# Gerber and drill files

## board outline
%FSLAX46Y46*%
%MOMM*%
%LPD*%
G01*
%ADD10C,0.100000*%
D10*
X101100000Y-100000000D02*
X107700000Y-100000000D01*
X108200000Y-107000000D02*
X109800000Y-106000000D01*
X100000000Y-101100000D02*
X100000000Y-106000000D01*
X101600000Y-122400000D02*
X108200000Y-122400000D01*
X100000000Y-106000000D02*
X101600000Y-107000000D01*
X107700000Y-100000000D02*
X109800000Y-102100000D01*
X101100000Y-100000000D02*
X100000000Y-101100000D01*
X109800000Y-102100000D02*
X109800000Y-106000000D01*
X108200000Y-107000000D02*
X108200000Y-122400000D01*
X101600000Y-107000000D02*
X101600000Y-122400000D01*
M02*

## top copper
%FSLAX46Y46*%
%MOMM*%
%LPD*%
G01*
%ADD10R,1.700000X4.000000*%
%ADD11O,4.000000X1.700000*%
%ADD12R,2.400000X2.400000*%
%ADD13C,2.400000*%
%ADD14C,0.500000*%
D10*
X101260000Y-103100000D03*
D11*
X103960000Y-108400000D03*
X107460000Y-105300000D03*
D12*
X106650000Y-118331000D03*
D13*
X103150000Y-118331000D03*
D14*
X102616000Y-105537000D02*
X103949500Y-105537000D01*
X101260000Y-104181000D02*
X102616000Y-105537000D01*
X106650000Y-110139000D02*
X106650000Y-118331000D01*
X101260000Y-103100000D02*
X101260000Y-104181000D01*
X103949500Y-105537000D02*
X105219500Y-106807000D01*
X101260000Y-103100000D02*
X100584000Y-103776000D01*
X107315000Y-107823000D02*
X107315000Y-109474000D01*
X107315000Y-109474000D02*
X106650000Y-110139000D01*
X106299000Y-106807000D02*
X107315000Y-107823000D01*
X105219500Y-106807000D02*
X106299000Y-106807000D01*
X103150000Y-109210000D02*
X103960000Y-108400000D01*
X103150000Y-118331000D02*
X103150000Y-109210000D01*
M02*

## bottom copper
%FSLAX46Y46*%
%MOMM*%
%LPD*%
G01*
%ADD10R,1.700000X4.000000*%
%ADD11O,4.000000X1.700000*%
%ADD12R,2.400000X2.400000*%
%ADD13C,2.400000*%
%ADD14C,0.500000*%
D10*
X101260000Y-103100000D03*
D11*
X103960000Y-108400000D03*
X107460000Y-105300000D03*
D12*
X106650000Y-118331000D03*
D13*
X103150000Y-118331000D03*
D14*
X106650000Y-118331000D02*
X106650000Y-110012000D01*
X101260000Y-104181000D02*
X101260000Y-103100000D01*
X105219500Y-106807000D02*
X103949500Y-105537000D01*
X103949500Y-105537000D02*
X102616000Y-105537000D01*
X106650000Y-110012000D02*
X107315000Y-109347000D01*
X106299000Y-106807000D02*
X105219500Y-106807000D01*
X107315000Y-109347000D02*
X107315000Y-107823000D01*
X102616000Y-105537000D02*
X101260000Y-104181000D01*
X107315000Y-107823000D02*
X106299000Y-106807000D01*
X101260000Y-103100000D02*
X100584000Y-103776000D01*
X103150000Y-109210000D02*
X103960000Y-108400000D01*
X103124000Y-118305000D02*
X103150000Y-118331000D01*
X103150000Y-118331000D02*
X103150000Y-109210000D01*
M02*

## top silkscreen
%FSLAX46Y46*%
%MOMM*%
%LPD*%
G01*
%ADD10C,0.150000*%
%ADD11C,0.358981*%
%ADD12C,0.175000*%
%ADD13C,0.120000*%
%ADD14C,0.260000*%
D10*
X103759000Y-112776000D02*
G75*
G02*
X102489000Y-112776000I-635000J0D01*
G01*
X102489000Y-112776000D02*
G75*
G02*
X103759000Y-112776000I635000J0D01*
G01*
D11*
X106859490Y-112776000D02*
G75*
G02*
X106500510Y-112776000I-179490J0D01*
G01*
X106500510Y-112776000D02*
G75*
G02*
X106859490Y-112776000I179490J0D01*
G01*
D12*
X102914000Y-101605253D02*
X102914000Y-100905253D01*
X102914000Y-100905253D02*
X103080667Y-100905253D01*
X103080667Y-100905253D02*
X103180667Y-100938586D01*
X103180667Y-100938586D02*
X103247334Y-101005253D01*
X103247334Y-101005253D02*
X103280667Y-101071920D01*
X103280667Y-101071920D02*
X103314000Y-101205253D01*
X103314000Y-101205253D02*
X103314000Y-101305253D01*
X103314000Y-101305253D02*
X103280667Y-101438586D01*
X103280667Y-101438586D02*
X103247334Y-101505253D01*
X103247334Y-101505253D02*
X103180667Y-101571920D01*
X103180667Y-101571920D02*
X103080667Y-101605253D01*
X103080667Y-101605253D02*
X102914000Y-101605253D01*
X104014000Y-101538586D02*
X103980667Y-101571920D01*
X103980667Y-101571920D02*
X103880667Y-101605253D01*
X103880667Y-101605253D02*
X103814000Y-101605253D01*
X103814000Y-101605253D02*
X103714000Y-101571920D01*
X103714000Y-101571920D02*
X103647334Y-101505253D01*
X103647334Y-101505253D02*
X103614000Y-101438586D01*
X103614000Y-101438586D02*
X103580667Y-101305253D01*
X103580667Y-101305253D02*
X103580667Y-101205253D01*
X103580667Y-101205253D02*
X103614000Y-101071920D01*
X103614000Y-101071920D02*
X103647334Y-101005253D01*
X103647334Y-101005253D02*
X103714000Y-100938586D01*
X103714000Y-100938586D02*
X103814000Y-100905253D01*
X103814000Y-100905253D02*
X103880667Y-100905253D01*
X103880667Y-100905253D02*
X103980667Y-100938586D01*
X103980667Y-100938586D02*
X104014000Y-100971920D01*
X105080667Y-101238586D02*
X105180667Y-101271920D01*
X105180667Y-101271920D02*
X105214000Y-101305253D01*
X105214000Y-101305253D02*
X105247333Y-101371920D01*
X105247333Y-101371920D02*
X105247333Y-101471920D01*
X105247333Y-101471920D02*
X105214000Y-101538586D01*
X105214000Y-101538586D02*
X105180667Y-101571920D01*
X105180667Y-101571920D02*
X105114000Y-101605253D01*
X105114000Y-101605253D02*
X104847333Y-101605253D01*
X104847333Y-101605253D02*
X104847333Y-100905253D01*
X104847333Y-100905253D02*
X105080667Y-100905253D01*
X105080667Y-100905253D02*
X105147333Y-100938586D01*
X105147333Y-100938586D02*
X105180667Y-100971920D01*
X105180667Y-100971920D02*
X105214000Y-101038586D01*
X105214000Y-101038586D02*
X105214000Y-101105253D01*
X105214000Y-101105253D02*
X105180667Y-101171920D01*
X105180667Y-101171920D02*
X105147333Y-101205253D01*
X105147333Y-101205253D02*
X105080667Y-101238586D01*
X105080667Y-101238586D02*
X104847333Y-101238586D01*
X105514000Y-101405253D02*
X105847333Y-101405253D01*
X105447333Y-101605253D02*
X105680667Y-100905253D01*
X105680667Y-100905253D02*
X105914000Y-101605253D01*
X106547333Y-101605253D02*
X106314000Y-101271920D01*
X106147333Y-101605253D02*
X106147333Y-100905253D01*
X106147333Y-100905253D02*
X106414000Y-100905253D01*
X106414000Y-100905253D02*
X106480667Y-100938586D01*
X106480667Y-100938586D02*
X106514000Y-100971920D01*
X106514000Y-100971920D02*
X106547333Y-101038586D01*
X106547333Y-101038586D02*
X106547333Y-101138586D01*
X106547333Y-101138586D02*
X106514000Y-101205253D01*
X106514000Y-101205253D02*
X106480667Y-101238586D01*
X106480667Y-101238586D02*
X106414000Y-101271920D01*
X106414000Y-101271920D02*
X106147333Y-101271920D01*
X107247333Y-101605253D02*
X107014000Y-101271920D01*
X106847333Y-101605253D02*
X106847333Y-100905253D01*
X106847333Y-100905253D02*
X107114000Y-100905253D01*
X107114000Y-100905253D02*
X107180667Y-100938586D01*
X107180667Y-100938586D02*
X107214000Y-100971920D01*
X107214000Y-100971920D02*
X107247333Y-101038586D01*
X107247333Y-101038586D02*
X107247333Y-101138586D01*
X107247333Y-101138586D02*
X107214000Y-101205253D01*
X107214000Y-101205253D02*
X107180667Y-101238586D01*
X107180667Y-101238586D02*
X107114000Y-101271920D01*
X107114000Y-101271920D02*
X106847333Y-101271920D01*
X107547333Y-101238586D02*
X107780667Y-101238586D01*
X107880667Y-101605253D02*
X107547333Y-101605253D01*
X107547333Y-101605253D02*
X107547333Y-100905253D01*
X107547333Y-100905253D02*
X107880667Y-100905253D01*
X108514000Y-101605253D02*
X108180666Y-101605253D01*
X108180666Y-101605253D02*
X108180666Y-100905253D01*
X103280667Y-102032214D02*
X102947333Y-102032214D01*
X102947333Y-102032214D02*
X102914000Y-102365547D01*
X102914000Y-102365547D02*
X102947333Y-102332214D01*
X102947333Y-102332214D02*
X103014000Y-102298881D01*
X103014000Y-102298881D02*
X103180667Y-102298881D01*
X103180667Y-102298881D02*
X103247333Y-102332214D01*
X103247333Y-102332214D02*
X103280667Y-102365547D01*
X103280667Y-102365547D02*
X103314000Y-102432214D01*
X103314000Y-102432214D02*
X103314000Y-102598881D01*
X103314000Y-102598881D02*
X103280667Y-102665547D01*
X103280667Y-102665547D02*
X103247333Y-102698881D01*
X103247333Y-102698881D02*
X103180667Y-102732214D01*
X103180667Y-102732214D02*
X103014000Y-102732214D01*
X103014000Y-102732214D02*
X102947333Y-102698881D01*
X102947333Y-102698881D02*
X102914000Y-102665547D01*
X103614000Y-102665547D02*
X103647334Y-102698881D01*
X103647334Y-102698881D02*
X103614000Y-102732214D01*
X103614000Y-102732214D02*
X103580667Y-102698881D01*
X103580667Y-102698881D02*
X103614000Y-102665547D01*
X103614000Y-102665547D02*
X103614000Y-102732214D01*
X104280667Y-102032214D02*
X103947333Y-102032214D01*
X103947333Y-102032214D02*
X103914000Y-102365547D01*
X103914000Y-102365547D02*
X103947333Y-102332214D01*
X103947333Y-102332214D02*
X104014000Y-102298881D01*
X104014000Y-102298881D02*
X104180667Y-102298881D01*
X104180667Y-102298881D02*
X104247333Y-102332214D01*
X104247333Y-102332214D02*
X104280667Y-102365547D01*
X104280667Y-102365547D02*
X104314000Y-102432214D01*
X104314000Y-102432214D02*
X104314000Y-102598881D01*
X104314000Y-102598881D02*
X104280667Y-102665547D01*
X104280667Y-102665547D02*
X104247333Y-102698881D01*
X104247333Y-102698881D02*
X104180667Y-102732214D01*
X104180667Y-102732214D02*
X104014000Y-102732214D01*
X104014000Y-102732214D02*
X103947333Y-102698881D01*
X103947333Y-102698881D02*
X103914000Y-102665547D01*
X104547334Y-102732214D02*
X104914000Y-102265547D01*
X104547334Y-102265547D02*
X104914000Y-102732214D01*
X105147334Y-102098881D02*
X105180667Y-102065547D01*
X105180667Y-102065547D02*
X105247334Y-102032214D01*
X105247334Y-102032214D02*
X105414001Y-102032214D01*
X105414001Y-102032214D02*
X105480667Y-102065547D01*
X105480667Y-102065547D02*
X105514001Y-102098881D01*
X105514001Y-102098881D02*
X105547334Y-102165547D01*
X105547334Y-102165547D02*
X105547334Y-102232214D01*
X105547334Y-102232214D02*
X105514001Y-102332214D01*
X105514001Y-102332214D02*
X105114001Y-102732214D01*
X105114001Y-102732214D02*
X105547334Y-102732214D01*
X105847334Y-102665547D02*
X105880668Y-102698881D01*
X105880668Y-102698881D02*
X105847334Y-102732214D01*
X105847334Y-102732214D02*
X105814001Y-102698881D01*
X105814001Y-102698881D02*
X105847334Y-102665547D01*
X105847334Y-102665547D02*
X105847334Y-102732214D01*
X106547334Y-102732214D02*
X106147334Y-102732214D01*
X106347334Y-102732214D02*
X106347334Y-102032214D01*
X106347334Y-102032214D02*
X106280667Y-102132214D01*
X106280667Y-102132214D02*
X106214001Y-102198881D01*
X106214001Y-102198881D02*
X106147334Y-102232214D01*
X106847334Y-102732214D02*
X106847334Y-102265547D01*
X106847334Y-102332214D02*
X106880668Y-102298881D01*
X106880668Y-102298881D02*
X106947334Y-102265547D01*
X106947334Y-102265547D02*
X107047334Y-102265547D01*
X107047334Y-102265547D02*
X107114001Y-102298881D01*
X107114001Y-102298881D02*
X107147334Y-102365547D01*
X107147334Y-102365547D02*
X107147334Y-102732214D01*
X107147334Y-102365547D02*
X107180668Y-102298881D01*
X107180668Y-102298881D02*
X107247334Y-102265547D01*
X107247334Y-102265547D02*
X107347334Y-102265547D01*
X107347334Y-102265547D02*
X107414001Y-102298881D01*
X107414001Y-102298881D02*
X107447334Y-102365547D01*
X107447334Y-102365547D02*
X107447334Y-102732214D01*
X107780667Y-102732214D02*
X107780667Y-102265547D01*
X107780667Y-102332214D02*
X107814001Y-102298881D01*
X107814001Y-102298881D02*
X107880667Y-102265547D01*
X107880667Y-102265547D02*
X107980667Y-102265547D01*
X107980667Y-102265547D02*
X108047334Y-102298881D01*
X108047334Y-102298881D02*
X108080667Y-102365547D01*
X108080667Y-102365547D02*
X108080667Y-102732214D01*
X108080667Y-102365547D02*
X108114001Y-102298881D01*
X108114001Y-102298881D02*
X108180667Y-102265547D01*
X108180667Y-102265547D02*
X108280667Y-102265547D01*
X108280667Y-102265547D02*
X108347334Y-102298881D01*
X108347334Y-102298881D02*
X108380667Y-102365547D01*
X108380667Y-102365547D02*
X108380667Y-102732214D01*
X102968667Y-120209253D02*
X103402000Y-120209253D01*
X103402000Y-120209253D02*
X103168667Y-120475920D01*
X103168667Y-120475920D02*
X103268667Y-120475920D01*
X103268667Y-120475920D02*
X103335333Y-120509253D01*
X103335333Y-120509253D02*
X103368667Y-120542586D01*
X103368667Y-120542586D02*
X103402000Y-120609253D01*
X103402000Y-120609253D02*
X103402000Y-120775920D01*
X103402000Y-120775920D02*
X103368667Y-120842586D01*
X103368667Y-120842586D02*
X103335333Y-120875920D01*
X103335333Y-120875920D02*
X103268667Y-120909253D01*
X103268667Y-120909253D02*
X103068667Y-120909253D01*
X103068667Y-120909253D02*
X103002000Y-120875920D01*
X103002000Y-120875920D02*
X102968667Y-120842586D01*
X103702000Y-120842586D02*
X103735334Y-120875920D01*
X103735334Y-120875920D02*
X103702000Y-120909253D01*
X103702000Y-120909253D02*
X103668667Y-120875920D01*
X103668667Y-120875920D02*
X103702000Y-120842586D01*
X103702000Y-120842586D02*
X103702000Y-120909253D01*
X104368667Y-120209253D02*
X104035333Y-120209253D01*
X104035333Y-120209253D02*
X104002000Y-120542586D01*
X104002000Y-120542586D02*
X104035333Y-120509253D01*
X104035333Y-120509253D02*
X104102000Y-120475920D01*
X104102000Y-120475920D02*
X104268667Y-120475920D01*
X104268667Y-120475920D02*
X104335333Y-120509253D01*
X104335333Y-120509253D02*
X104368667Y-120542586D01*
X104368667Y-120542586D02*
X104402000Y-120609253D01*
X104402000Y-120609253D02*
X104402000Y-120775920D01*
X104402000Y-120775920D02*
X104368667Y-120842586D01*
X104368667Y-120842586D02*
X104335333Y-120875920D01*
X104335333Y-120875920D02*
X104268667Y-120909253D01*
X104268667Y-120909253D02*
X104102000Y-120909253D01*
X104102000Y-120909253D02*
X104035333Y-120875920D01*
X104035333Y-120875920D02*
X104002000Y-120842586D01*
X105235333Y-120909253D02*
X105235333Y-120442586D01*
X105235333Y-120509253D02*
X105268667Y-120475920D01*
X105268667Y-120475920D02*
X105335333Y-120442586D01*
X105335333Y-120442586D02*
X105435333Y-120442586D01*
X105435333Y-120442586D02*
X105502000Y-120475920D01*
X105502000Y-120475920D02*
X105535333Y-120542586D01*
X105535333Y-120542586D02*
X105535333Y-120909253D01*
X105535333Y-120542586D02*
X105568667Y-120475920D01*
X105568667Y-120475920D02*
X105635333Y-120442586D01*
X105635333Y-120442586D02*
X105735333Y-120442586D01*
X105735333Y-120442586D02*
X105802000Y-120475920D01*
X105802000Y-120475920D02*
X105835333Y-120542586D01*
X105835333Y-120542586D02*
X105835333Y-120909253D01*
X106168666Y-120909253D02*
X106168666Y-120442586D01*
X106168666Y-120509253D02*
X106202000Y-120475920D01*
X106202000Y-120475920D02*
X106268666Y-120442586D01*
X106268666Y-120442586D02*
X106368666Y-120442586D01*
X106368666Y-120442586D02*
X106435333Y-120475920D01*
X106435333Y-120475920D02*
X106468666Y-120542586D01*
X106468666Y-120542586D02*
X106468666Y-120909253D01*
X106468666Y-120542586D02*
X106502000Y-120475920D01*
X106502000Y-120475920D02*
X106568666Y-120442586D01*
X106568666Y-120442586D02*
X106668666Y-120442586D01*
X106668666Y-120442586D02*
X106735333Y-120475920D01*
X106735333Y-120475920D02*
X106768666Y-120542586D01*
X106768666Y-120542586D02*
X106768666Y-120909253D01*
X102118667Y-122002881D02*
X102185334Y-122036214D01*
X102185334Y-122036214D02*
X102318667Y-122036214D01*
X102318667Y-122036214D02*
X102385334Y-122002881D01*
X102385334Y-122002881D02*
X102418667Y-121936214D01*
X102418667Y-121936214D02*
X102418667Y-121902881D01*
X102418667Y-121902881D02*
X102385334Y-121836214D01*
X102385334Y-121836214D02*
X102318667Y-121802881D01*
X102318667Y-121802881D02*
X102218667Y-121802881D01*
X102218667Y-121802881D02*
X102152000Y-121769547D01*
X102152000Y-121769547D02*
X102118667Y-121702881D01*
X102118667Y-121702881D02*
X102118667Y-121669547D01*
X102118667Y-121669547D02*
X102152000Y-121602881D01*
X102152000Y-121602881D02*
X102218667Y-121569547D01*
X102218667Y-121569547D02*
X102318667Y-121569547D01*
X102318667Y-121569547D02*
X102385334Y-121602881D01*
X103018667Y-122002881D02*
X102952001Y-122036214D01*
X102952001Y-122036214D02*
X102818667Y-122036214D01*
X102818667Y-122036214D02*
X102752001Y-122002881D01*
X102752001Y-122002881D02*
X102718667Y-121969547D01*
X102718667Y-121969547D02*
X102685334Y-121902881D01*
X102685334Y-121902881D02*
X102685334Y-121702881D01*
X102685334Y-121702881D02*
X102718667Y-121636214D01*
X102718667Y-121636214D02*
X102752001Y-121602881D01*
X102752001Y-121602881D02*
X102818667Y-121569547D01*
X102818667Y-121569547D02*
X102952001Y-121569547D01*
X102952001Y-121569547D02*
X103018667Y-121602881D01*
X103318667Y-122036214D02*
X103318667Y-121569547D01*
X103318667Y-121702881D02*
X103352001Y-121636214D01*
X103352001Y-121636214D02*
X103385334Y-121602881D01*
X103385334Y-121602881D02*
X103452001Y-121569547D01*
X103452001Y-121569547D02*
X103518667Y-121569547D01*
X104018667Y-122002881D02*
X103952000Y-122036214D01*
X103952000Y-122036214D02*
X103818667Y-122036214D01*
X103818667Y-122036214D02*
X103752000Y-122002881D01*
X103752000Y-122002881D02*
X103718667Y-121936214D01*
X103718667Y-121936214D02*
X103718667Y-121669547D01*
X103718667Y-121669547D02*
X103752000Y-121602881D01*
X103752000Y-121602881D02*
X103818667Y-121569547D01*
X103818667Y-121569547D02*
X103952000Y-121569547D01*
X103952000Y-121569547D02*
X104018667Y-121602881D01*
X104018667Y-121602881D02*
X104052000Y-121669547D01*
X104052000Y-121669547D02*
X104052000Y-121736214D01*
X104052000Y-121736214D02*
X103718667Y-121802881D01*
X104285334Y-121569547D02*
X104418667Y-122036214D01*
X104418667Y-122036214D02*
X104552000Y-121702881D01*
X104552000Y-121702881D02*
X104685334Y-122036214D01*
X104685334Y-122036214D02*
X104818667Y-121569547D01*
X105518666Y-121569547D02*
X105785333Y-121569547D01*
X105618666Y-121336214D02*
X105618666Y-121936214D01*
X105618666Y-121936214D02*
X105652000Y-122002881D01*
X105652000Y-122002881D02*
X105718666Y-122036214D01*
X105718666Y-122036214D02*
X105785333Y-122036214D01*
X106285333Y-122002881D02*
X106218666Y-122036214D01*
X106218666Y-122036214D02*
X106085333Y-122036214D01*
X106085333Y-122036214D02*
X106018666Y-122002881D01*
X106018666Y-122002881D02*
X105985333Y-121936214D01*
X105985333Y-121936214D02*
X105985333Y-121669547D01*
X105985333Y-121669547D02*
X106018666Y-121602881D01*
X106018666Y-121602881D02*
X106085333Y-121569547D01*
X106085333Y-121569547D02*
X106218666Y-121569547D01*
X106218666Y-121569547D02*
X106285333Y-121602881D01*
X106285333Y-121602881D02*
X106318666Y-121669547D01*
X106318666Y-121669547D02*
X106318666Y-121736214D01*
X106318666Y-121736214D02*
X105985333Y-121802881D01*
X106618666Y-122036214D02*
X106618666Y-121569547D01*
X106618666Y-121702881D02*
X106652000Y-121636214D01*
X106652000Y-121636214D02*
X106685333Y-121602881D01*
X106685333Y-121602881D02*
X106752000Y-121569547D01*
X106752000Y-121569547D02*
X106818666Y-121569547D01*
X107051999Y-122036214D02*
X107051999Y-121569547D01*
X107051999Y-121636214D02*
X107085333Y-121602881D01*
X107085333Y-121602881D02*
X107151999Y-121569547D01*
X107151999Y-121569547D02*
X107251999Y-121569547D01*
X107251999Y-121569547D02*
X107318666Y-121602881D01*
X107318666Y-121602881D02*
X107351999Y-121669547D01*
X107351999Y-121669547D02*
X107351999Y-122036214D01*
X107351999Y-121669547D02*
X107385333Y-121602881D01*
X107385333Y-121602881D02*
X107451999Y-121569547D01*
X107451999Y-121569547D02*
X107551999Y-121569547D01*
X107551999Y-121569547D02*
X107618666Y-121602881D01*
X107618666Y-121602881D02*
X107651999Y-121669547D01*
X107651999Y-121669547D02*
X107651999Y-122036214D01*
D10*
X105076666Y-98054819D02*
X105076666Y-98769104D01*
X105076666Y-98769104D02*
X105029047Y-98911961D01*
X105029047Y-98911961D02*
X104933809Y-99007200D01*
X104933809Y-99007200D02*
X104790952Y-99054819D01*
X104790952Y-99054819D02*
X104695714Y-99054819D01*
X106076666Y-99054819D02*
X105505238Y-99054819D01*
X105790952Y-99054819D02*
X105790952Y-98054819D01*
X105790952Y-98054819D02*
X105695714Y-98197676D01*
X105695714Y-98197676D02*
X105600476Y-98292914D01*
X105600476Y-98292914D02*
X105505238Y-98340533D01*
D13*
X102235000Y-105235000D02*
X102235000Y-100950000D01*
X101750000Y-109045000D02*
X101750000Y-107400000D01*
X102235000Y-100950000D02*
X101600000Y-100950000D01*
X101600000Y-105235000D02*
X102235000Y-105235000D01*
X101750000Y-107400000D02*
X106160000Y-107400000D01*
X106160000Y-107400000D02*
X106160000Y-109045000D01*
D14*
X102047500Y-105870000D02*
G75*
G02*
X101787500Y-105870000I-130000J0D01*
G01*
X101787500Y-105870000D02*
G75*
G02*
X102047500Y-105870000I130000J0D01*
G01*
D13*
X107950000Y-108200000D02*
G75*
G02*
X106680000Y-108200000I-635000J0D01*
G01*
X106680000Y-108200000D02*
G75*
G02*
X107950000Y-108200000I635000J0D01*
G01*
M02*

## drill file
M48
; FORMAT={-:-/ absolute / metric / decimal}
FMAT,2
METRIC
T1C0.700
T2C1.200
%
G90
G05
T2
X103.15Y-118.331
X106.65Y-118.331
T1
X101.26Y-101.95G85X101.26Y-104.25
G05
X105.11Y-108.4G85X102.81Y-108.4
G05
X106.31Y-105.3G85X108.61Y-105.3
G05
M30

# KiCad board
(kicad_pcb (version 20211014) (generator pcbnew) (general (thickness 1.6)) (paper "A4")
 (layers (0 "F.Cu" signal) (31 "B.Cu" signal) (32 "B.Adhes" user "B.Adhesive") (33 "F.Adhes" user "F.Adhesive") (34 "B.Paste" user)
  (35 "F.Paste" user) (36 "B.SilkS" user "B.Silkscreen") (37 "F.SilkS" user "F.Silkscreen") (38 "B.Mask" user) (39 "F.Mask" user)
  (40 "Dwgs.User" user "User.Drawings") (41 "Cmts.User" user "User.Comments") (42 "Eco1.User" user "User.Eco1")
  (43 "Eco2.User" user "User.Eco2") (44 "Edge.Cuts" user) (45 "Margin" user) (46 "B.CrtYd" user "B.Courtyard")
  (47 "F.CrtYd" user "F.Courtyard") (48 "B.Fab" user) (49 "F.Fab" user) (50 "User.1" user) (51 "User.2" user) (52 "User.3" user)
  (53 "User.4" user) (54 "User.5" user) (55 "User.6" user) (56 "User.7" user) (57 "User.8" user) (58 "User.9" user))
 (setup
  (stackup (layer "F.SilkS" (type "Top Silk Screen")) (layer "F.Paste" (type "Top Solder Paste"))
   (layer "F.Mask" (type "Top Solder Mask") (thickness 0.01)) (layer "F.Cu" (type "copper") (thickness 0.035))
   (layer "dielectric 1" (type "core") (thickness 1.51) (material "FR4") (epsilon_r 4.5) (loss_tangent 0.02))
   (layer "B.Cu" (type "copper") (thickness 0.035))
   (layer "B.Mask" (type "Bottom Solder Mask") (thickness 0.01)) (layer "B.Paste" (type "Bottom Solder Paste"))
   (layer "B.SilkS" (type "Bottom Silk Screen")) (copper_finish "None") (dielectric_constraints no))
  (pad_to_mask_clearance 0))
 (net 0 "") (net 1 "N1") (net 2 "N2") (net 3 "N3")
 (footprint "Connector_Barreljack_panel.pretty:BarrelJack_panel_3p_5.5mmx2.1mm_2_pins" (layer "F.Cu") (at 105.41 104.6)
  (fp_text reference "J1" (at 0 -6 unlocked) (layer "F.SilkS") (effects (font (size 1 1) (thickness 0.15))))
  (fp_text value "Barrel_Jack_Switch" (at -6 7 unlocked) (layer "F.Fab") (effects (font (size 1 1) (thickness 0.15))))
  (fp_line (start -3.175 0.635) (end -3.175 -3.65) (layer "F.SilkS") (width 0.12))
  (fp_line (start -3.66 4.445) (end -3.66 2.8) (layer "F.SilkS") (width 0.12))
  (fp_line (start -3.175 -3.65) (end -3.81 -3.65) (layer "F.SilkS") (width 0.12))
  (fp_line (start -3.81 0.635) (end -3.175 0.635) (layer "F.SilkS") (width 0.12))
  (fp_line (start -3.66 2.8) (end 0.75 2.8) (layer "F.SilkS") (width 0.12))
  (fp_line (start 0.75 2.8) (end 0.75 4.445) (layer "F.SilkS") (width 0.12))
  (fp_circle (center -3.4925 1.27) (end -3.2925 1.27) (layer "F.SilkS") (width 0.12) (fill solid))
  (fp_circle (center 1.905 3.6) (end 2.54 3.6) (layer "F.SilkS") (width 0.12) (fill none))
  (pad "1" thru_hole rect (at -4.15 -1.5) (size 1.7 4) (drill oval 0.7 3) (layers *.Cu *.Mask) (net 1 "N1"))
  (pad "2" thru_hole oval (at -1.45 3.8 270) (size 1.7 4) (drill oval 0.7 3) (layers *.Cu *.Mask) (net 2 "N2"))
  (pad "3" thru_hole oval (at 2.05 0.7 90) (size 1.7 4) (drill oval 0.7 3) (layers *.Cu *.Mask) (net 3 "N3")))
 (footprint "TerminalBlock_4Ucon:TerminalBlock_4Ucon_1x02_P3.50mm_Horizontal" (layer "B.Cu") (at 106.65 118.331 180)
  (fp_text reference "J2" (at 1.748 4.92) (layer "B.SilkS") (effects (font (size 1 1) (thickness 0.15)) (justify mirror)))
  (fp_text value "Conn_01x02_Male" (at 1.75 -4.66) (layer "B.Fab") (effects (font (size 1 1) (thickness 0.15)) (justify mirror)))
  (pad "1" thru_hole rect (at 0 0 180) (size 2.4 2.4) (drill 1.2) (layers *.Cu *.Mask) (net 1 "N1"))
  (pad "2" thru_hole circle (at 3.5 0 180) (size 2.4 2.4) (drill 1.2) (layers *.Cu *.Mask) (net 2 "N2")))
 (gr_circle (center 103.124 112.776) (end 103.632 112.395) (layer "F.SilkS") (width 0.15) (fill none))
 (gr_circle (center 106.68 112.776) (end 106.963981 112.776) (layer "F.SilkS") (width 0.15) (fill solid))
 (gr_line (start 101.1 100) (end 107.7 100) (layer "Edge.Cuts") (width 0.1))
 (gr_line (start 108.2 107) (end 109.8 106) (layer "Edge.Cuts") (width 0.1))
 (gr_line (start 100 101.1) (end 100 106) (layer "Edge.Cuts") (width 0.1))
 (gr_line (start 101.6 122.4) (end 108.2 122.4) (layer "Edge.Cuts") (width 0.1))
 (gr_line (start 100 106) (end 101.6 107) (layer "Edge.Cuts") (width 0.1))
 (gr_line (start 107.7 100) (end 109.8 102.1) (layer "Edge.Cuts") (width 0.1))
 (gr_line (start 101.1 100) (end 100 101.1) (layer "Edge.Cuts") (width 0.1))
 (gr_line (start 109.8 102.1) (end 109.8 106) (layer "Edge.Cuts") (width 0.1))
 (gr_line (start 108.2 107) (end 108.2 122.4) (layer "Edge.Cuts") (width 0.1))
 (gr_line (start 101.6 107) (end 101.6 122.4) (layer "Edge.Cuts") (width 0.1))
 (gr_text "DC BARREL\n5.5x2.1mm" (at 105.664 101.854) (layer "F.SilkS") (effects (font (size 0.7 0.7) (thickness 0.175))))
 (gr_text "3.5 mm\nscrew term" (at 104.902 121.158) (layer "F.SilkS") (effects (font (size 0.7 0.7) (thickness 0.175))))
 (segment (start 102.616 105.537) (end 103.9495 105.537) (width 0.5) (layer "F.Cu") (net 1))
 (segment (start 101.26 104.181) (end 102.616 105.537) (width 0.5) (layer "F.Cu") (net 1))
 (segment (start 106.65 110.139) (end 106.65 118.331) (width 0.5) (layer "F.Cu") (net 1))
 (segment (start 101.26 103.1) (end 101.26 104.181) (width 0.5) (layer "F.Cu") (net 1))
 (segment (start 103.9495 105.537) (end 105.2195 106.807) (width 0.5) (layer "F.Cu") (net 1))
 (segment (start 101.26 103.1) (end 100.584 103.776) (width 0.5) (layer "F.Cu") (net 1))
 (segment (start 107.315 107.823) (end 107.315 109.474) (width 0.5) (layer "F.Cu") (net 1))
 (segment (start 107.315 109.474) (end 106.65 110.139) (width 0.5) (layer "F.Cu") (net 1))
 (segment (start 106.299 106.807) (end 107.315 107.823) (width 0.5) (layer "F.Cu") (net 1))
 (segment (start 105.2195 106.807) (end 106.299 106.807) (width 0.5) (layer "F.Cu") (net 1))
 (segment (start 106.65 118.331) (end 106.65 110.012) (width 0.5) (layer "B.Cu") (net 1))
 (segment (start 101.26 104.181) (end 101.26 103.1) (width 0.5) (layer "B.Cu") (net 1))
 (segment (start 105.2195 106.807) (end 103.9495 105.537) (width 0.5) (layer "B.Cu") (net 1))
 (segment (start 103.9495 105.537) (end 102.616 105.537) (width 0.5) (layer "B.Cu") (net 1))
 (segment (start 106.65 110.012) (end 107.315 109.347) (width 0.5) (layer "B.Cu") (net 1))
 (segment (start 106.299 106.807) (end 105.2195 106.807) (width 0.5) (layer "B.Cu") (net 1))
 (segment (start 107.315 109.347) (end 107.315 107.823) (width 0.5) (layer "B.Cu") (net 1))
 (segment (start 102.616 105.537) (end 101.26 104.181) (width 0.5) (layer "B.Cu") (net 1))
 (segment (start 107.315 107.823) (end 106.299 106.807) (width 0.5) (layer "B.Cu") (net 1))
 (segment (start 101.26 103.1) (end 100.584 103.776) (width 0.5) (layer "B.Cu") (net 1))
 (segment (start 103.15 109.21) (end 103.96 108.4) (width 0.5) (layer "F.Cu") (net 2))
 (segment (start 103.15 118.331) (end 103.15 109.21) (width 0.5) (layer "F.Cu") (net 2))
 (segment (start 103.15 109.21) (end 103.96 108.4) (width 0.5) (layer "B.Cu") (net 2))
 (segment (start 103.124 118.305) (end 103.15 118.331) (width 0.5) (layer "B.Cu") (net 2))
 (segment (start 103.15 118.331) (end 103.15 109.21) (width 0.5) (layer "B.Cu") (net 2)))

